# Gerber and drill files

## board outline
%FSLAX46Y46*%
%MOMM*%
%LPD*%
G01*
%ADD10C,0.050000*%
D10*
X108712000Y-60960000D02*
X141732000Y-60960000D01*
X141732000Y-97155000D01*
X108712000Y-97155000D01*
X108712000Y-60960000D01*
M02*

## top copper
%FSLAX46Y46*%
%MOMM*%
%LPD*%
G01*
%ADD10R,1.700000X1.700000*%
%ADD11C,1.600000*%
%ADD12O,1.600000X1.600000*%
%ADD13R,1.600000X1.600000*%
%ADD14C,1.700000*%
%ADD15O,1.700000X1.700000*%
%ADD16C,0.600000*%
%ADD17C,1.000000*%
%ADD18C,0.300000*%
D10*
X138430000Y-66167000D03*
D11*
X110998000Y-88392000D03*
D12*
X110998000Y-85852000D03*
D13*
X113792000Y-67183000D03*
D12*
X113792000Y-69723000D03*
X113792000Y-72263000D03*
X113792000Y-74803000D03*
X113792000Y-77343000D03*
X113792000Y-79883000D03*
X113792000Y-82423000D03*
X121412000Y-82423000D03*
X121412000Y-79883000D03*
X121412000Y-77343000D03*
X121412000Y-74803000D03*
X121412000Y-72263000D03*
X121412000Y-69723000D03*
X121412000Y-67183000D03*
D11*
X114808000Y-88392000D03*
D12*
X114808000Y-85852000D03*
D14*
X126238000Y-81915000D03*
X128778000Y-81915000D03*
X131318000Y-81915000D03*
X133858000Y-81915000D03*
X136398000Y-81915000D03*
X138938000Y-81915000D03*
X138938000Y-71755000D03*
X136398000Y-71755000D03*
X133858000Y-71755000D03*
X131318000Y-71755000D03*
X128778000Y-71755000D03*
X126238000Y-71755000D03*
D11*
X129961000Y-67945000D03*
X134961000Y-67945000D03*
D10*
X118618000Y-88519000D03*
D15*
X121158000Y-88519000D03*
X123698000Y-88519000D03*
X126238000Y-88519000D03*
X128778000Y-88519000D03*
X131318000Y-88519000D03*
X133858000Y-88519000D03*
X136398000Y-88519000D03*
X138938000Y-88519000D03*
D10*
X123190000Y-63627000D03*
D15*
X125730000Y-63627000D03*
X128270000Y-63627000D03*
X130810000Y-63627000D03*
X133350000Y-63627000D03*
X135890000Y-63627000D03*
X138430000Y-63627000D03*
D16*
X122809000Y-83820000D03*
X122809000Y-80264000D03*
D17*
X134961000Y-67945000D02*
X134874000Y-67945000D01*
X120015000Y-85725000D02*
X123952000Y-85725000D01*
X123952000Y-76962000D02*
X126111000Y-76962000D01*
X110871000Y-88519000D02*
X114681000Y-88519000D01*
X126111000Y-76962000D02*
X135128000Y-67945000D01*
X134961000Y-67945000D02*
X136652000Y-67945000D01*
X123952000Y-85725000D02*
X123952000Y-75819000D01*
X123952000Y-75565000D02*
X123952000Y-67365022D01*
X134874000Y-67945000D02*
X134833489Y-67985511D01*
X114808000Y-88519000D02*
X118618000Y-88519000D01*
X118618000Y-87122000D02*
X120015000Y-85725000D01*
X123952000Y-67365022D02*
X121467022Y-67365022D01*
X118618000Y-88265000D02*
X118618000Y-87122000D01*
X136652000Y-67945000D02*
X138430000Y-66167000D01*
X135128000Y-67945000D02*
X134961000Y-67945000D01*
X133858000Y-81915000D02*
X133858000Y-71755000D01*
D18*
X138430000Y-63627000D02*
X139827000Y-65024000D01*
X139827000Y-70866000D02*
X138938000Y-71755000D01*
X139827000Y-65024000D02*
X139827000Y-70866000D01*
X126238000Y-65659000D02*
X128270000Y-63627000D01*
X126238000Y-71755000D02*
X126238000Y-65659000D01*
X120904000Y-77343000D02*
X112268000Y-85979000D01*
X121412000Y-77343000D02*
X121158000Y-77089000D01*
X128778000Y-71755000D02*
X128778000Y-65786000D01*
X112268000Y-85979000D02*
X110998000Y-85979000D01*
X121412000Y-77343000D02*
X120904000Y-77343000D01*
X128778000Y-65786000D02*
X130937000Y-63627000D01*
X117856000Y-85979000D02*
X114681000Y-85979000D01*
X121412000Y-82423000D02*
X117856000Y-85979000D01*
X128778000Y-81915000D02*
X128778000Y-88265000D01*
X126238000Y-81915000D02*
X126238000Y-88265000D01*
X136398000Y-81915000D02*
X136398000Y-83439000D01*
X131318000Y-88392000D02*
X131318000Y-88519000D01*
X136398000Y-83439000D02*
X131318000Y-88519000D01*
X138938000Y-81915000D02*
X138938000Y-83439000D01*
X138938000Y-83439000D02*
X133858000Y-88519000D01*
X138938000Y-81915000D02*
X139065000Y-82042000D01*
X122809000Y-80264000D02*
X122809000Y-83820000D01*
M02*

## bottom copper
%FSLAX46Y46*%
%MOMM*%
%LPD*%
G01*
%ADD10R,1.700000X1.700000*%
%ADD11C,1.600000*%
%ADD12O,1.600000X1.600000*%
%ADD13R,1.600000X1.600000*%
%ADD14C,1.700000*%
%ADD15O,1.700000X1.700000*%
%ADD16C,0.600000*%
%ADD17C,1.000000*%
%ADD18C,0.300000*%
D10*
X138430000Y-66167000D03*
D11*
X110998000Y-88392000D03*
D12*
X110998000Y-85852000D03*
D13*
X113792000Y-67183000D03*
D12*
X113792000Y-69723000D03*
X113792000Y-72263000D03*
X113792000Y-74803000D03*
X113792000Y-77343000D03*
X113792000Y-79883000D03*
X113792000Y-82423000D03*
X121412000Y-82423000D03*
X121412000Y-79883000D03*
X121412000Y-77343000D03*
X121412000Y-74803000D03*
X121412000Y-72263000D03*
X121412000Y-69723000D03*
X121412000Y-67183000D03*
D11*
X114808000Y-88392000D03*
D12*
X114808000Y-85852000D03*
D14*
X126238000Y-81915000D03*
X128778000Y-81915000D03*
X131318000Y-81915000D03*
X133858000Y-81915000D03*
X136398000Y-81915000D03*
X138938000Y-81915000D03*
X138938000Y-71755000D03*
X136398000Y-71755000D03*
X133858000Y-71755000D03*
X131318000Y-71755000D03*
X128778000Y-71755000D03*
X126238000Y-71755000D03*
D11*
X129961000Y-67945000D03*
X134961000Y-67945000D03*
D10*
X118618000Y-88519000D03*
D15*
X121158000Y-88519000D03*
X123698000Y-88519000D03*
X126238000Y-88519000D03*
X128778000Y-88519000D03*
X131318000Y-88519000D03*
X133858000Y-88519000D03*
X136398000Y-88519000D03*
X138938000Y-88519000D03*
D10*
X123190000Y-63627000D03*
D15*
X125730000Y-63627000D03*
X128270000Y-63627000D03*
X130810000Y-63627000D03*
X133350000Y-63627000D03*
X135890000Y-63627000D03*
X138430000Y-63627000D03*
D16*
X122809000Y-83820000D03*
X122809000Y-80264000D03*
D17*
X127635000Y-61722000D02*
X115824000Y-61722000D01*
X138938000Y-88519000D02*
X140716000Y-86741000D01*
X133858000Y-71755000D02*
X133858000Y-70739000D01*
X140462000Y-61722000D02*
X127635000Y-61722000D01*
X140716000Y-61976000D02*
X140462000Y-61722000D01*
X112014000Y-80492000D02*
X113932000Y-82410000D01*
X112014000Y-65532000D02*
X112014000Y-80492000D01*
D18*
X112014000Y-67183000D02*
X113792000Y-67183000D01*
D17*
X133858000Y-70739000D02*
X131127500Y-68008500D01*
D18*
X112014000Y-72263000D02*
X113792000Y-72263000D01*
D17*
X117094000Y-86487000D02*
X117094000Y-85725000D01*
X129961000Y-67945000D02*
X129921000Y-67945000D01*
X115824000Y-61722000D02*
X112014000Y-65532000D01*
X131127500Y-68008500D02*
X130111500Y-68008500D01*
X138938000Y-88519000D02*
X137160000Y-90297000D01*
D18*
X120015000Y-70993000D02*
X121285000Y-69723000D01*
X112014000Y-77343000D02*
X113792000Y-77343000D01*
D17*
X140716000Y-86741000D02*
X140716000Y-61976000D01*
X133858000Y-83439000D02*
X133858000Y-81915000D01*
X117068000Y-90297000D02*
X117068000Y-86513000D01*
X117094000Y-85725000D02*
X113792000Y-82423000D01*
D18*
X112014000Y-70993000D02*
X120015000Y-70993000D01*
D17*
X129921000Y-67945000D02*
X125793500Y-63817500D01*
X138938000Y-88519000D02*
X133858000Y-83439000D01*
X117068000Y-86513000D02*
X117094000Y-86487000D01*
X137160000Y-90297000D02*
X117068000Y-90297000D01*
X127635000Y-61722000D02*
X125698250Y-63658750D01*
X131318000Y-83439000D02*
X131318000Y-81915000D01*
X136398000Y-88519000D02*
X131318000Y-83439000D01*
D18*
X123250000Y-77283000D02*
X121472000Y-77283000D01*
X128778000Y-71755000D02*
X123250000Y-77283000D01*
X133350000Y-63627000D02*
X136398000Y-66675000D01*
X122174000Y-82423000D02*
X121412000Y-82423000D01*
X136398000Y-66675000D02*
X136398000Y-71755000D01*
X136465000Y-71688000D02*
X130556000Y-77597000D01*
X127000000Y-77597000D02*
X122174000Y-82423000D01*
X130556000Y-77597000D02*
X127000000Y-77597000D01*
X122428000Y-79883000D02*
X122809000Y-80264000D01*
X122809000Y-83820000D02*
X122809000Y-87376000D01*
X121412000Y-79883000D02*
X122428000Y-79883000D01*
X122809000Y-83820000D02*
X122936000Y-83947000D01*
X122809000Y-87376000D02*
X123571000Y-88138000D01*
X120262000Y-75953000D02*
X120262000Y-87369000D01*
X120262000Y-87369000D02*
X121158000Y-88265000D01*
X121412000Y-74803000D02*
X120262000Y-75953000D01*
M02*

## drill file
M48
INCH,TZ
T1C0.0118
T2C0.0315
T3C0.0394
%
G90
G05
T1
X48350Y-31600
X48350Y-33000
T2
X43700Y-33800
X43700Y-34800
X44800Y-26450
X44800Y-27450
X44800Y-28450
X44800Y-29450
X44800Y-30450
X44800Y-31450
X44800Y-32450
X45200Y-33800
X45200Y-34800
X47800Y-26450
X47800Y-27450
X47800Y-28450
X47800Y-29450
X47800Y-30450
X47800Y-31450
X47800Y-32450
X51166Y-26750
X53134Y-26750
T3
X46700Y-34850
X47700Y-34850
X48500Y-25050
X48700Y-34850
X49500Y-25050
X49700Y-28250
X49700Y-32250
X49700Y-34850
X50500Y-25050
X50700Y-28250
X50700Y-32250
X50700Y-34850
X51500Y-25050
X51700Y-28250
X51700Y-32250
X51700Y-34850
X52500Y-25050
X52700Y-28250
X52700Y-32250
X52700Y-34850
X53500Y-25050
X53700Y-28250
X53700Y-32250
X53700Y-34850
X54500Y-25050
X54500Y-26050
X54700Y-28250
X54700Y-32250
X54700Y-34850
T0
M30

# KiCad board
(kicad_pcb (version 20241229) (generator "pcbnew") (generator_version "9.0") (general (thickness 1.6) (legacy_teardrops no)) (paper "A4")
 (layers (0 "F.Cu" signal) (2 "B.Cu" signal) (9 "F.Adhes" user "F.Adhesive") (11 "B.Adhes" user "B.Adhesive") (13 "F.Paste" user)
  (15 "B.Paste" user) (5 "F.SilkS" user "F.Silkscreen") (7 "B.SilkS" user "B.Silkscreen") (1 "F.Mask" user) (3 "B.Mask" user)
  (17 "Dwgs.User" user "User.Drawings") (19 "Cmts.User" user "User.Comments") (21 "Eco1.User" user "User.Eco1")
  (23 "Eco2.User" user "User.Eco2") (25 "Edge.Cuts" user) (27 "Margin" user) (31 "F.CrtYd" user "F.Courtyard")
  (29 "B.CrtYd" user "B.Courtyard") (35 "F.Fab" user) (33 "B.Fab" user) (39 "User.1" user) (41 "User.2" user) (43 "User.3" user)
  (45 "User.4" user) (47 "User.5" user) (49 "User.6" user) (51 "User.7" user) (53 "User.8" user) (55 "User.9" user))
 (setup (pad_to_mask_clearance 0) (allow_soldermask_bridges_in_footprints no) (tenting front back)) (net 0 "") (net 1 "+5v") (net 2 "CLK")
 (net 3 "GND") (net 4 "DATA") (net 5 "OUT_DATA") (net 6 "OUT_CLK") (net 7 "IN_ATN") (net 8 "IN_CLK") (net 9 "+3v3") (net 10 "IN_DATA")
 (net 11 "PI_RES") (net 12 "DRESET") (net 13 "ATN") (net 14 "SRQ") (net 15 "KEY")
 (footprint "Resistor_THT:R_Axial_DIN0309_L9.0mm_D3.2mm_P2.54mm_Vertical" (layer "F.Cu") (at 110.998 88.392 90)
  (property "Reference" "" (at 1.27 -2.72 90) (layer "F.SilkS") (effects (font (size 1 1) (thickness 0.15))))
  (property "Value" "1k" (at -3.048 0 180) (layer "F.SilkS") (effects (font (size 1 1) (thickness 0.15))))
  (pad "1" thru_hole circle (at 0 0 90) (size 1.6 1.6) (drill 0.8) (layers "*.Cu" "*.Mask") (remove_unused_layers no) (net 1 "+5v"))
  (pad "2" thru_hole oval (at 2.54 0 90) (size 1.6 1.6) (drill 0.8) (layers "*.Cu" "*.Mask") (remove_unused_layers no) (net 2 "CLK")))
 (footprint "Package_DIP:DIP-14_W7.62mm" (layer "F.Cu") (at 113.792 67.183)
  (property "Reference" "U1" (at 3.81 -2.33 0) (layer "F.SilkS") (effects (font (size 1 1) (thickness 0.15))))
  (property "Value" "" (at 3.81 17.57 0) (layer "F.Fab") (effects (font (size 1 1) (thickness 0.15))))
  (pad "1" thru_hole rect (at 0 0) (size 1.6 1.6) (drill 0.8) (layers "*.Cu" "*.Mask") (remove_unused_layers no) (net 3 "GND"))
  (pad "2" thru_hole oval (at 0 2.54) (size 1.6 1.6) (drill 0.8) (layers "*.Cu" "*.Mask") (remove_unused_layers no))
  (pad "3" thru_hole oval (at 0 5.08) (size 1.6 1.6) (drill 0.8) (layers "*.Cu" "*.Mask") (remove_unused_layers no) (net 3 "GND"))
  (pad "4" thru_hole oval (at 0 7.62) (size 1.6 1.6) (drill 0.8) (layers "*.Cu" "*.Mask") (remove_unused_layers no))
  (pad "5" thru_hole oval (at 0 10.16) (size 1.6 1.6) (drill 0.8) (layers "*.Cu" "*.Mask") (remove_unused_layers no) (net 3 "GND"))
  (pad "6" thru_hole oval (at 0 12.7) (size 1.6 1.6) (drill 0.8) (layers "*.Cu" "*.Mask") (remove_unused_layers no))
  (pad "7" thru_hole oval (at 0 15.24) (size 1.6 1.6) (drill 0.8) (layers "*.Cu" "*.Mask") (remove_unused_layers no) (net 3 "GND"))
  (pad "8" thru_hole oval (at 7.62 15.24) (size 1.6 1.6) (drill 0.8) (layers "*.Cu" "*.Mask") (remove_unused_layers no) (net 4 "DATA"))
  (pad "9" thru_hole oval (at 7.62 12.7) (size 1.6 1.6) (drill 0.8) (layers "*.Cu" "*.Mask") (remove_unused_layers no) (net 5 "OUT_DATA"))
  (pad "10" thru_hole oval (at 7.62 10.16) (size 1.6 1.6) (drill 0.8) (layers "*.Cu" "*.Mask") (remove_unused_layers no) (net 2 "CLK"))
  (pad "11" thru_hole oval (at 7.62 7.62) (size 1.6 1.6) (drill 0.8) (layers "*.Cu" "*.Mask") (remove_unused_layers no) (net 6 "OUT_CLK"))
  (pad "12" thru_hole oval (at 7.62 5.08) (size 1.6 1.6) (drill 0.8) (layers "*.Cu" "*.Mask") (remove_unused_layers no))
  (pad "13" thru_hole oval (at 7.62 2.54) (size 1.6 1.6) (drill 0.8) (layers "*.Cu" "*.Mask") (remove_unused_layers no) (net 3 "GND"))
  (pad "14" thru_hole oval (at 7.62 0) (size 1.6 1.6) (drill 0.8) (layers "*.Cu" "*.Mask") (remove_unused_layers no) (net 1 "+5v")))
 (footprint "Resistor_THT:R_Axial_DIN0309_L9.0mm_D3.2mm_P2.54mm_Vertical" (layer "F.Cu") (at 114.808 88.392 90)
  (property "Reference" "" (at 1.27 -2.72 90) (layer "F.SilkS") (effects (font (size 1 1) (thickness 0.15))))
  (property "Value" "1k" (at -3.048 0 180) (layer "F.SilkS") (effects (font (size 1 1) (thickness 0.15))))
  (pad "1" thru_hole circle (at 0 0 90) (size 1.6 1.6) (drill 0.8) (layers "*.Cu" "*.Mask") (remove_unused_layers no) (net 1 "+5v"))
  (pad "2" thru_hole oval (at 2.54 0 90) (size 1.6 1.6) (drill 0.8) (layers "*.Cu" "*.Mask") (remove_unused_layers no) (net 4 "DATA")))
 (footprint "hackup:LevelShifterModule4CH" (layer "F.Cu") (at 133.858 76.835 90)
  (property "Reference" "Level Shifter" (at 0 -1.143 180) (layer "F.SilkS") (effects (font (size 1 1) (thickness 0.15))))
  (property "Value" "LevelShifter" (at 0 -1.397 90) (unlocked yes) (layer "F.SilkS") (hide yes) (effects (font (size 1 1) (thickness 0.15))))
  (pad "1" thru_hole circle (at -5.08 -7.62 90) (size 1.7 1.7) (drill 1) (layers "*.Cu" "*.Mask") (remove_unused_layers no) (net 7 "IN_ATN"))
  (pad "2" thru_hole circle (at -5.08 -5.08 90) (size 1.7 1.7) (drill 1) (layers "*.Cu" "*.Mask") (remove_unused_layers no) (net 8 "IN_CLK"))
  (pad "3" thru_hole circle (at -5.08 -2.54 90) (size 1.7 1.7) (drill 1) (layers "*.Cu" "*.Mask") (remove_unused_layers no) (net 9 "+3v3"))
  (pad "4" thru_hole circle (at -5.08 0 90) (size 1.7 1.7) (drill 1) (layers "*.Cu" "*.Mask") (remove_unused_layers no) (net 3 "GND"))
  (pad "5" thru_hole circle (at -5.08 2.54 90) (size 1.7 1.7) (drill 1) (layers "*.Cu" "*.Mask") (remove_unused_layers no)
   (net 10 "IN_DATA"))
  (pad "6" thru_hole circle (at -5.08 5.08 90) (size 1.7 1.7) (drill 1) (layers "*.Cu" "*.Mask") (remove_unused_layers no) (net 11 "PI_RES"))
  (pad "7" thru_hole circle (at 5.08 5.08 90) (size 1.7 1.7) (drill 1) (layers "*.Cu" "*.Mask") (remove_unused_layers no) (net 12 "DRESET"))
  (pad "8" thru_hole circle (at 5.08 2.54 90) (size 1.7 1.7) (drill 1) (layers "*.Cu" "*.Mask") (remove_unused_layers no) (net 4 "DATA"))
  (pad "9" thru_hole circle (at 5.08 0 90) (size 1.7 1.7) (drill 1) (layers "*.Cu" "*.Mask") (remove_unused_layers no) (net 3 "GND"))
  (pad "10" thru_hole circle (at 5.08 -2.54 90) (size 1.7 1.7) (drill 1) (layers "*.Cu" "*.Mask") (remove_unused_layers no) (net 1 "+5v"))
  (pad "11" thru_hole circle (at 5.08 -5.08 90) (size 1.7 1.7) (drill 1) (layers "*.Cu" "*.Mask") (remove_unused_layers no) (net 2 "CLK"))
  (pad "12" thru_hole circle (at 5.08 -7.62 90) (size 1.7 1.7) (drill 1) (layers "*.Cu" "*.Mask") (remove_unused_layers no) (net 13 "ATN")))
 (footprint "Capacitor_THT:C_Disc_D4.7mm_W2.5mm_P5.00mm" (layer "F.Cu") (at 129.961 67.945)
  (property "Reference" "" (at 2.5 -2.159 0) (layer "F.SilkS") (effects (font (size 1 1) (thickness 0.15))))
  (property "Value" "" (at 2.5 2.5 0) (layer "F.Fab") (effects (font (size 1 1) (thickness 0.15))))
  (pad "1" thru_hole circle (at 0 0) (size 1.6 1.6) (drill 0.8) (layers "*.Cu" "*.Mask") (remove_unused_layers no) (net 3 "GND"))
  (pad "2" thru_hole circle (at 5 0) (size 1.6 1.6) (drill 0.8) (layers "*.Cu" "*.Mask") (remove_unused_layers no) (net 1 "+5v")))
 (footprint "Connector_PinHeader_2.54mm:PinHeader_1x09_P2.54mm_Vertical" (layer "F.Cu") (at 118.618 88.519 90)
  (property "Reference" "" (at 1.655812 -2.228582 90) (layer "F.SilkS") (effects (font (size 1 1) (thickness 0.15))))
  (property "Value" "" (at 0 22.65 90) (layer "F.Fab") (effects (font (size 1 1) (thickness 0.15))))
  (pad "1" thru_hole rect (at 0 0 90) (size 1.7 1.7) (drill 1) (layers "*.Cu" "*.Mask") (remove_unused_layers no) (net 1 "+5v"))
  (pad "2" thru_hole oval (at 0 2.54 90) (size 1.7 1.7) (drill 1) (layers "*.Cu" "*.Mask") (remove_unused_layers no) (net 6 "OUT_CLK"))
  (pad "3" thru_hole oval (at 0 5.08 90) (size 1.7 1.7) (drill 1) (layers "*.Cu" "*.Mask") (remove_unused_layers no) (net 5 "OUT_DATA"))
  (pad "4" thru_hole oval (at 0 7.62 90) (size 1.7 1.7) (drill 1) (layers "*.Cu" "*.Mask") (remove_unused_layers no) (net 7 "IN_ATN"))
  (pad "5" thru_hole oval (at 0 10.16 90) (size 1.7 1.7) (drill 1) (layers "*.Cu" "*.Mask") (remove_unused_layers no) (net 8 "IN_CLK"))
  (pad "6" thru_hole oval (at 0 12.7 90) (size 1.7 1.7) (drill 1) (layers "*.Cu" "*.Mask") (remove_unused_layers no) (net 10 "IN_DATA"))
  (pad "7" thru_hole oval (at 0 15.24 90) (size 1.7 1.7) (drill 1) (layers "*.Cu" "*.Mask") (remove_unused_layers no) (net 11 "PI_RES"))
  (pad "8" thru_hole oval (at 0 17.78 90) (size 1.7 1.7) (drill 1) (layers "*.Cu" "*.Mask") (remove_unused_layers no) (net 9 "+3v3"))
  (pad "9" thru_hole oval (at 0 20.32 90) (size 1.7 1.7) (drill 1) (layers "*.Cu" "*.Mask") (remove_unused_layers no) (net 3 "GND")))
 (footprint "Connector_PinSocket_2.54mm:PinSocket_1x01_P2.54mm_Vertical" (layer "B.Cu") (at 138.43 66.167 180)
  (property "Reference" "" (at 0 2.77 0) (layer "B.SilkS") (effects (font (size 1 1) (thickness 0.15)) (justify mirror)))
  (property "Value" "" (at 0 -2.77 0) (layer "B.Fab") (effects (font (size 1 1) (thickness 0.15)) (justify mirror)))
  (pad "1" thru_hole rect (at 0 0 180) (size 1.7 1.7) (drill 1) (layers "*.Cu" "*.Mask") (remove_unused_layers no) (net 1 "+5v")))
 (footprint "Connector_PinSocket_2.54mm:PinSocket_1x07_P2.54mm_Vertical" (layer "B.Cu") (at 123.19 63.627 -90)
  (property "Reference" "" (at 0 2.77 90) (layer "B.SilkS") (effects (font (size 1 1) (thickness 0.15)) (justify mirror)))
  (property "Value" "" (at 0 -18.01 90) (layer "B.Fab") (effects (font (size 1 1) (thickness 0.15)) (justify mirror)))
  (pad "1" thru_hole rect (at 0 0 270) (size 1.7 1.7) (drill 1) (layers "*.Cu" "*.Mask") (remove_unused_layers no) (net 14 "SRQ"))
  (pad "2" thru_hole oval (at 0 -2.54 270) (size 1.7 1.7) (drill 1) (layers "*.Cu" "*.Mask") (remove_unused_layers no) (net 3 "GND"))
  (pad "3" thru_hole oval (at 0 -5.08 270) (size 1.7 1.7) (drill 1) (layers "*.Cu" "*.Mask") (remove_unused_layers no) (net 13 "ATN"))
  (pad "4" thru_hole oval (at 0 -7.62 270) (size 1.7 1.7) (drill 1) (layers "*.Cu" "*.Mask") (remove_unused_layers no) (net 2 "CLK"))
  (pad "5" thru_hole oval (at 0 -10.16 270) (size 1.7 1.7) (drill 1) (layers "*.Cu" "*.Mask") (remove_unused_layers no) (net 4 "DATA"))
  (pad "6" thru_hole oval (at 0 -12.7 270) (size 1.7 1.7) (drill 1) (layers "*.Cu" "*.Mask") (remove_unused_layers no) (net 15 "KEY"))
  (pad "7" thru_hole oval (at 0 -15.24 270) (size 1.7 1.7) (drill 1) (layers "*.Cu" "*.Mask") (remove_unused_layers no) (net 12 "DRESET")))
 (gr_rect (start 108.712 60.96) (end 141.732 97.155) (stroke (width 0.05) (type default)) (fill no) (layer "Edge.Cuts"))
 (segment (start 134.961 67.945) (end 134.874 67.945) (width 1) (layer "F.Cu") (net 1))
 (segment (start 120.015 85.725) (end 123.952 85.725) (width 1) (layer "F.Cu") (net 1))
 (segment (start 123.952 76.962) (end 126.111 76.962) (width 1) (layer "F.Cu") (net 1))
 (segment (start 110.871 88.519) (end 114.681 88.519) (width 1) (layer "F.Cu") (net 1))
 (segment (start 126.111 76.962) (end 135.128 67.945) (width 1) (layer "F.Cu") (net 1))
 (segment (start 134.961 67.945) (end 136.652 67.945) (width 1) (layer "F.Cu") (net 1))
 (segment (start 123.952 85.725) (end 123.952 75.819) (width 1) (layer "F.Cu") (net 1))
 (segment (start 123.952 75.565) (end 123.952 67.365022) (width 1) (layer "F.Cu") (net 1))
 (segment (start 134.874 67.945) (end 134.833489 67.985511) (width 1) (layer "F.Cu") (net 1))
 (segment (start 114.808 88.519) (end 118.618 88.519) (width 1) (layer "F.Cu") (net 1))
 (segment (start 118.618 87.122) (end 120.015 85.725) (width 1) (layer "F.Cu") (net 1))
 (segment (start 123.952 67.365022) (end 121.467022 67.365022) (width 1) (layer "F.Cu") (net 1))
 (segment (start 118.618 88.265) (end 118.618 87.122) (width 1) (layer "F.Cu") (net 1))
 (segment (start 136.652 67.945) (end 138.43 66.167) (width 1) (layer "F.Cu") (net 1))
 (segment (start 135.128 67.945) (end 134.961 67.945) (width 1) (layer "F.Cu") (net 1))
 (segment (start 133.858 81.915) (end 133.858 71.755) (width 1) (layer "F.Cu") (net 3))
 (segment (start 127.635 61.722) (end 115.824 61.722) (width 1) (layer "B.Cu") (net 3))
 (segment (start 138.938 88.519) (end 140.716 86.741) (width 1) (layer "B.Cu") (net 3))
 (segment (start 133.858 71.755) (end 133.858 70.739) (width 1) (layer "B.Cu") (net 3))
 (segment (start 140.462 61.722) (end 127.635 61.722) (width 1) (layer "B.Cu") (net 3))
 (segment (start 140.716 61.976) (end 140.462 61.722) (width 1) (layer "B.Cu") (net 3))
 (segment (start 112.014 80.492) (end 113.932 82.41) (width 1) (layer "B.Cu") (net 3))
 (segment (start 112.014 65.532) (end 112.014 80.492) (width 1) (layer "B.Cu") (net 3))
 (segment (start 112.014 67.183) (end 113.792 67.183) (width 0.3) (layer "B.Cu") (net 3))
 (segment (start 133.858 70.739) (end 131.1275 68.0085) (width 1) (layer "B.Cu") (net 3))
 (segment (start 112.014 72.263) (end 113.792 72.263) (width 0.3) (layer "B.Cu") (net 3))
 (segment (start 117.094 86.487) (end 117.094 85.725) (width 1) (layer "B.Cu") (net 3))
 (segment (start 129.961 67.945) (end 129.921 67.945) (width 1) (layer "B.Cu") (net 3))
 (segment (start 115.824 61.722) (end 112.014 65.532) (width 1) (layer "B.Cu") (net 3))
 (segment (start 131.1275 68.0085) (end 130.1115 68.0085) (width 1) (layer "B.Cu") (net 3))
 (segment (start 138.938 88.519) (end 137.16 90.297) (width 1) (layer "B.Cu") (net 3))
 (segment (start 120.015 70.993) (end 121.285 69.723) (width 0.3) (layer "B.Cu") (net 3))
 (segment (start 112.014 77.343) (end 113.792 77.343) (width 0.3) (layer "B.Cu") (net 3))
 (segment (start 140.716 86.741) (end 140.716 61.976) (width 1) (layer "B.Cu") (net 3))
 (segment (start 133.858 83.439) (end 133.858 81.915) (width 1) (layer "B.Cu") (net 3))
 (segment (start 117.068 90.297) (end 117.068 86.513) (width 1) (layer "B.Cu") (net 3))
 (segment (start 117.094 85.725) (end 113.792 82.423) (width 1) (layer "B.Cu") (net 3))
 (segment (start 112.014 70.993) (end 120.015 70.993) (width 0.3) (layer "B.Cu") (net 3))
 (segment (start 129.921 67.945) (end 125.7935 63.8175) (width 1) (layer "B.Cu") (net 3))
 (segment (start 138.938 88.519) (end 133.858 83.439) (width 1) (layer "B.Cu") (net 3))
 (segment (start 117.068 86.513) (end 117.094 86.487) (width 1) (layer "B.Cu") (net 3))
 (segment (start 137.16 90.297) (end 117.068 90.297) (width 1) (layer "B.Cu") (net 3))
 (segment (start 127.635 61.722) (end 125.69825 63.65875) (width 1) (layer "B.Cu") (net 3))
 (segment (start 131.318 83.439) (end 131.318 81.915) (width 1) (layer "B.Cu") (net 9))
 (segment (start 136.398 88.519) (end 131.318 83.439) (width 1) (layer "B.Cu") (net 9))
 (segment (start 138.43 63.627) (end 139.827 65.024) (width 0.3) (layer "F.Cu") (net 12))
 (segment (start 139.827 70.866) (end 138.938 71.755) (width 0.3) (layer "F.Cu") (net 12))
 (segment (start 139.827 65.024) (end 139.827 70.866) (width 0.3) (layer "F.Cu") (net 12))
 (segment (start 126.238 65.659) (end 128.27 63.627) (width 0.3) (layer "F.Cu") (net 13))
 (segment (start 126.238 71.755) (end 126.238 65.659) (width 0.3) (layer "F.Cu") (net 13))
 (segment (start 120.904 77.343) (end 112.268 85.979) (width 0.3) (layer "F.Cu") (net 2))
 (segment (start 121.412 77.343) (end 121.158 77.089) (width 0.3) (layer "F.Cu") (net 2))
 (segment (start 128.778 71.755) (end 128.778 65.786) (width 0.3) (layer "F.Cu") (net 2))
 (segment (start 112.268 85.979) (end 110.998 85.979) (width 0.3) (layer "F.Cu") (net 2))
 (segment (start 121.412 77.343) (end 120.904 77.343) (width 0.3) (layer "F.Cu") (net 2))
 (segment (start 128.778 65.786) (end 130.937 63.627) (width 0.3) (layer "F.Cu") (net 2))
 (segment (start 123.25 77.283) (end 121.472 77.283) (width 0.3) (layer "B.Cu") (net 2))
 (segment (start 128.778 71.755) (end 123.25 77.283) (width 0.3) (layer "B.Cu") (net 2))
 (segment (start 117.856 85.979) (end 114.681 85.979) (width 0.3) (layer "F.Cu") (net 4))
 (segment (start 121.412 82.423) (end 117.856 85.979) (width 0.3) (layer "F.Cu") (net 4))
 (segment (start 133.35 63.627) (end 136.398 66.675) (width 0.3) (layer "B.Cu") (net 4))
 (segment (start 122.174 82.423) (end 121.412 82.423) (width 0.3) (layer "B.Cu") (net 4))
 (segment (start 136.398 66.675) (end 136.398 71.755) (width 0.3) (layer "B.Cu") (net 4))
 (segment (start 136.465 71.688) (end 130.556 77.597) (width 0.3) (layer "B.Cu") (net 4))
 (segment (start 127 77.597) (end 122.174 82.423) (width 0.3) (layer "B.Cu") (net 4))
 (segment (start 130.556 77.597) (end 127 77.597) (width 0.3) (layer "B.Cu") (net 4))
 (segment (start 128.778 81.915) (end 128.778 88.265) (width 0.3) (layer "F.Cu") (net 8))
 (segment (start 126.238 81.915) (end 126.238 88.265) (width 0.3) (layer "F.Cu") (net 7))
 (segment (start 136.398 81.915) (end 136.398 83.439) (width 0.3) (layer "F.Cu") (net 10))
 (segment (start 131.318 88.392) (end 131.318 88.519) (width 0.3) (layer "F.Cu") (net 10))
 (segment (start 136.398 83.439) (end 131.318 88.519) (width 0.3) (layer "F.Cu") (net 10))
 (segment (start 138.938 81.915) (end 138.938 83.439) (width 0.3) (layer "F.Cu") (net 11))
 (segment (start 138.938 83.439) (end 133.858 88.519) (width 0.3) (layer "F.Cu") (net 11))
 (segment (start 138.938 81.915) (end 139.065 82.042) (width 0.3) (layer "F.Cu") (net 11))
 (segment (start 122.809 80.264) (end 122.809 83.82) (width 0.3) (layer "F.Cu") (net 5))
 (via (at 122.809 83.82) (size 0.6) (drill 0.3) (layers "F.Cu" "B.Cu") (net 5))
 (via (at 122.809 80.264) (size 0.6) (drill 0.3) (layers "F.Cu" "B.Cu") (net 5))
 (segment (start 122.428 79.883) (end 122.809 80.264) (width 0.3) (layer "B.Cu") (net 5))
 (segment (start 122.809 83.82) (end 122.809 87.376) (width 0.3) (layer "B.Cu") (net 5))
 (segment (start 121.412 79.883) (end 122.428 79.883) (width 0.3) (layer "B.Cu") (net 5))
 (segment (start 122.809 83.82) (end 122.936 83.947) (width 0.3) (layer "B.Cu") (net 5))
 (segment (start 122.809 87.376) (end 123.571 88.138) (width 0.3) (layer "B.Cu") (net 5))
 (segment (start 120.262 75.953) (end 120.262 87.369) (width 0.3) (layer "B.Cu") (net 6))
 (segment (start 120.262 87.369) (end 121.158 88.265) (width 0.3) (layer "B.Cu") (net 6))
 (segment (start 121.412 74.803) (end 120.262 75.953) (width 0.3) (layer "B.Cu") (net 6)))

